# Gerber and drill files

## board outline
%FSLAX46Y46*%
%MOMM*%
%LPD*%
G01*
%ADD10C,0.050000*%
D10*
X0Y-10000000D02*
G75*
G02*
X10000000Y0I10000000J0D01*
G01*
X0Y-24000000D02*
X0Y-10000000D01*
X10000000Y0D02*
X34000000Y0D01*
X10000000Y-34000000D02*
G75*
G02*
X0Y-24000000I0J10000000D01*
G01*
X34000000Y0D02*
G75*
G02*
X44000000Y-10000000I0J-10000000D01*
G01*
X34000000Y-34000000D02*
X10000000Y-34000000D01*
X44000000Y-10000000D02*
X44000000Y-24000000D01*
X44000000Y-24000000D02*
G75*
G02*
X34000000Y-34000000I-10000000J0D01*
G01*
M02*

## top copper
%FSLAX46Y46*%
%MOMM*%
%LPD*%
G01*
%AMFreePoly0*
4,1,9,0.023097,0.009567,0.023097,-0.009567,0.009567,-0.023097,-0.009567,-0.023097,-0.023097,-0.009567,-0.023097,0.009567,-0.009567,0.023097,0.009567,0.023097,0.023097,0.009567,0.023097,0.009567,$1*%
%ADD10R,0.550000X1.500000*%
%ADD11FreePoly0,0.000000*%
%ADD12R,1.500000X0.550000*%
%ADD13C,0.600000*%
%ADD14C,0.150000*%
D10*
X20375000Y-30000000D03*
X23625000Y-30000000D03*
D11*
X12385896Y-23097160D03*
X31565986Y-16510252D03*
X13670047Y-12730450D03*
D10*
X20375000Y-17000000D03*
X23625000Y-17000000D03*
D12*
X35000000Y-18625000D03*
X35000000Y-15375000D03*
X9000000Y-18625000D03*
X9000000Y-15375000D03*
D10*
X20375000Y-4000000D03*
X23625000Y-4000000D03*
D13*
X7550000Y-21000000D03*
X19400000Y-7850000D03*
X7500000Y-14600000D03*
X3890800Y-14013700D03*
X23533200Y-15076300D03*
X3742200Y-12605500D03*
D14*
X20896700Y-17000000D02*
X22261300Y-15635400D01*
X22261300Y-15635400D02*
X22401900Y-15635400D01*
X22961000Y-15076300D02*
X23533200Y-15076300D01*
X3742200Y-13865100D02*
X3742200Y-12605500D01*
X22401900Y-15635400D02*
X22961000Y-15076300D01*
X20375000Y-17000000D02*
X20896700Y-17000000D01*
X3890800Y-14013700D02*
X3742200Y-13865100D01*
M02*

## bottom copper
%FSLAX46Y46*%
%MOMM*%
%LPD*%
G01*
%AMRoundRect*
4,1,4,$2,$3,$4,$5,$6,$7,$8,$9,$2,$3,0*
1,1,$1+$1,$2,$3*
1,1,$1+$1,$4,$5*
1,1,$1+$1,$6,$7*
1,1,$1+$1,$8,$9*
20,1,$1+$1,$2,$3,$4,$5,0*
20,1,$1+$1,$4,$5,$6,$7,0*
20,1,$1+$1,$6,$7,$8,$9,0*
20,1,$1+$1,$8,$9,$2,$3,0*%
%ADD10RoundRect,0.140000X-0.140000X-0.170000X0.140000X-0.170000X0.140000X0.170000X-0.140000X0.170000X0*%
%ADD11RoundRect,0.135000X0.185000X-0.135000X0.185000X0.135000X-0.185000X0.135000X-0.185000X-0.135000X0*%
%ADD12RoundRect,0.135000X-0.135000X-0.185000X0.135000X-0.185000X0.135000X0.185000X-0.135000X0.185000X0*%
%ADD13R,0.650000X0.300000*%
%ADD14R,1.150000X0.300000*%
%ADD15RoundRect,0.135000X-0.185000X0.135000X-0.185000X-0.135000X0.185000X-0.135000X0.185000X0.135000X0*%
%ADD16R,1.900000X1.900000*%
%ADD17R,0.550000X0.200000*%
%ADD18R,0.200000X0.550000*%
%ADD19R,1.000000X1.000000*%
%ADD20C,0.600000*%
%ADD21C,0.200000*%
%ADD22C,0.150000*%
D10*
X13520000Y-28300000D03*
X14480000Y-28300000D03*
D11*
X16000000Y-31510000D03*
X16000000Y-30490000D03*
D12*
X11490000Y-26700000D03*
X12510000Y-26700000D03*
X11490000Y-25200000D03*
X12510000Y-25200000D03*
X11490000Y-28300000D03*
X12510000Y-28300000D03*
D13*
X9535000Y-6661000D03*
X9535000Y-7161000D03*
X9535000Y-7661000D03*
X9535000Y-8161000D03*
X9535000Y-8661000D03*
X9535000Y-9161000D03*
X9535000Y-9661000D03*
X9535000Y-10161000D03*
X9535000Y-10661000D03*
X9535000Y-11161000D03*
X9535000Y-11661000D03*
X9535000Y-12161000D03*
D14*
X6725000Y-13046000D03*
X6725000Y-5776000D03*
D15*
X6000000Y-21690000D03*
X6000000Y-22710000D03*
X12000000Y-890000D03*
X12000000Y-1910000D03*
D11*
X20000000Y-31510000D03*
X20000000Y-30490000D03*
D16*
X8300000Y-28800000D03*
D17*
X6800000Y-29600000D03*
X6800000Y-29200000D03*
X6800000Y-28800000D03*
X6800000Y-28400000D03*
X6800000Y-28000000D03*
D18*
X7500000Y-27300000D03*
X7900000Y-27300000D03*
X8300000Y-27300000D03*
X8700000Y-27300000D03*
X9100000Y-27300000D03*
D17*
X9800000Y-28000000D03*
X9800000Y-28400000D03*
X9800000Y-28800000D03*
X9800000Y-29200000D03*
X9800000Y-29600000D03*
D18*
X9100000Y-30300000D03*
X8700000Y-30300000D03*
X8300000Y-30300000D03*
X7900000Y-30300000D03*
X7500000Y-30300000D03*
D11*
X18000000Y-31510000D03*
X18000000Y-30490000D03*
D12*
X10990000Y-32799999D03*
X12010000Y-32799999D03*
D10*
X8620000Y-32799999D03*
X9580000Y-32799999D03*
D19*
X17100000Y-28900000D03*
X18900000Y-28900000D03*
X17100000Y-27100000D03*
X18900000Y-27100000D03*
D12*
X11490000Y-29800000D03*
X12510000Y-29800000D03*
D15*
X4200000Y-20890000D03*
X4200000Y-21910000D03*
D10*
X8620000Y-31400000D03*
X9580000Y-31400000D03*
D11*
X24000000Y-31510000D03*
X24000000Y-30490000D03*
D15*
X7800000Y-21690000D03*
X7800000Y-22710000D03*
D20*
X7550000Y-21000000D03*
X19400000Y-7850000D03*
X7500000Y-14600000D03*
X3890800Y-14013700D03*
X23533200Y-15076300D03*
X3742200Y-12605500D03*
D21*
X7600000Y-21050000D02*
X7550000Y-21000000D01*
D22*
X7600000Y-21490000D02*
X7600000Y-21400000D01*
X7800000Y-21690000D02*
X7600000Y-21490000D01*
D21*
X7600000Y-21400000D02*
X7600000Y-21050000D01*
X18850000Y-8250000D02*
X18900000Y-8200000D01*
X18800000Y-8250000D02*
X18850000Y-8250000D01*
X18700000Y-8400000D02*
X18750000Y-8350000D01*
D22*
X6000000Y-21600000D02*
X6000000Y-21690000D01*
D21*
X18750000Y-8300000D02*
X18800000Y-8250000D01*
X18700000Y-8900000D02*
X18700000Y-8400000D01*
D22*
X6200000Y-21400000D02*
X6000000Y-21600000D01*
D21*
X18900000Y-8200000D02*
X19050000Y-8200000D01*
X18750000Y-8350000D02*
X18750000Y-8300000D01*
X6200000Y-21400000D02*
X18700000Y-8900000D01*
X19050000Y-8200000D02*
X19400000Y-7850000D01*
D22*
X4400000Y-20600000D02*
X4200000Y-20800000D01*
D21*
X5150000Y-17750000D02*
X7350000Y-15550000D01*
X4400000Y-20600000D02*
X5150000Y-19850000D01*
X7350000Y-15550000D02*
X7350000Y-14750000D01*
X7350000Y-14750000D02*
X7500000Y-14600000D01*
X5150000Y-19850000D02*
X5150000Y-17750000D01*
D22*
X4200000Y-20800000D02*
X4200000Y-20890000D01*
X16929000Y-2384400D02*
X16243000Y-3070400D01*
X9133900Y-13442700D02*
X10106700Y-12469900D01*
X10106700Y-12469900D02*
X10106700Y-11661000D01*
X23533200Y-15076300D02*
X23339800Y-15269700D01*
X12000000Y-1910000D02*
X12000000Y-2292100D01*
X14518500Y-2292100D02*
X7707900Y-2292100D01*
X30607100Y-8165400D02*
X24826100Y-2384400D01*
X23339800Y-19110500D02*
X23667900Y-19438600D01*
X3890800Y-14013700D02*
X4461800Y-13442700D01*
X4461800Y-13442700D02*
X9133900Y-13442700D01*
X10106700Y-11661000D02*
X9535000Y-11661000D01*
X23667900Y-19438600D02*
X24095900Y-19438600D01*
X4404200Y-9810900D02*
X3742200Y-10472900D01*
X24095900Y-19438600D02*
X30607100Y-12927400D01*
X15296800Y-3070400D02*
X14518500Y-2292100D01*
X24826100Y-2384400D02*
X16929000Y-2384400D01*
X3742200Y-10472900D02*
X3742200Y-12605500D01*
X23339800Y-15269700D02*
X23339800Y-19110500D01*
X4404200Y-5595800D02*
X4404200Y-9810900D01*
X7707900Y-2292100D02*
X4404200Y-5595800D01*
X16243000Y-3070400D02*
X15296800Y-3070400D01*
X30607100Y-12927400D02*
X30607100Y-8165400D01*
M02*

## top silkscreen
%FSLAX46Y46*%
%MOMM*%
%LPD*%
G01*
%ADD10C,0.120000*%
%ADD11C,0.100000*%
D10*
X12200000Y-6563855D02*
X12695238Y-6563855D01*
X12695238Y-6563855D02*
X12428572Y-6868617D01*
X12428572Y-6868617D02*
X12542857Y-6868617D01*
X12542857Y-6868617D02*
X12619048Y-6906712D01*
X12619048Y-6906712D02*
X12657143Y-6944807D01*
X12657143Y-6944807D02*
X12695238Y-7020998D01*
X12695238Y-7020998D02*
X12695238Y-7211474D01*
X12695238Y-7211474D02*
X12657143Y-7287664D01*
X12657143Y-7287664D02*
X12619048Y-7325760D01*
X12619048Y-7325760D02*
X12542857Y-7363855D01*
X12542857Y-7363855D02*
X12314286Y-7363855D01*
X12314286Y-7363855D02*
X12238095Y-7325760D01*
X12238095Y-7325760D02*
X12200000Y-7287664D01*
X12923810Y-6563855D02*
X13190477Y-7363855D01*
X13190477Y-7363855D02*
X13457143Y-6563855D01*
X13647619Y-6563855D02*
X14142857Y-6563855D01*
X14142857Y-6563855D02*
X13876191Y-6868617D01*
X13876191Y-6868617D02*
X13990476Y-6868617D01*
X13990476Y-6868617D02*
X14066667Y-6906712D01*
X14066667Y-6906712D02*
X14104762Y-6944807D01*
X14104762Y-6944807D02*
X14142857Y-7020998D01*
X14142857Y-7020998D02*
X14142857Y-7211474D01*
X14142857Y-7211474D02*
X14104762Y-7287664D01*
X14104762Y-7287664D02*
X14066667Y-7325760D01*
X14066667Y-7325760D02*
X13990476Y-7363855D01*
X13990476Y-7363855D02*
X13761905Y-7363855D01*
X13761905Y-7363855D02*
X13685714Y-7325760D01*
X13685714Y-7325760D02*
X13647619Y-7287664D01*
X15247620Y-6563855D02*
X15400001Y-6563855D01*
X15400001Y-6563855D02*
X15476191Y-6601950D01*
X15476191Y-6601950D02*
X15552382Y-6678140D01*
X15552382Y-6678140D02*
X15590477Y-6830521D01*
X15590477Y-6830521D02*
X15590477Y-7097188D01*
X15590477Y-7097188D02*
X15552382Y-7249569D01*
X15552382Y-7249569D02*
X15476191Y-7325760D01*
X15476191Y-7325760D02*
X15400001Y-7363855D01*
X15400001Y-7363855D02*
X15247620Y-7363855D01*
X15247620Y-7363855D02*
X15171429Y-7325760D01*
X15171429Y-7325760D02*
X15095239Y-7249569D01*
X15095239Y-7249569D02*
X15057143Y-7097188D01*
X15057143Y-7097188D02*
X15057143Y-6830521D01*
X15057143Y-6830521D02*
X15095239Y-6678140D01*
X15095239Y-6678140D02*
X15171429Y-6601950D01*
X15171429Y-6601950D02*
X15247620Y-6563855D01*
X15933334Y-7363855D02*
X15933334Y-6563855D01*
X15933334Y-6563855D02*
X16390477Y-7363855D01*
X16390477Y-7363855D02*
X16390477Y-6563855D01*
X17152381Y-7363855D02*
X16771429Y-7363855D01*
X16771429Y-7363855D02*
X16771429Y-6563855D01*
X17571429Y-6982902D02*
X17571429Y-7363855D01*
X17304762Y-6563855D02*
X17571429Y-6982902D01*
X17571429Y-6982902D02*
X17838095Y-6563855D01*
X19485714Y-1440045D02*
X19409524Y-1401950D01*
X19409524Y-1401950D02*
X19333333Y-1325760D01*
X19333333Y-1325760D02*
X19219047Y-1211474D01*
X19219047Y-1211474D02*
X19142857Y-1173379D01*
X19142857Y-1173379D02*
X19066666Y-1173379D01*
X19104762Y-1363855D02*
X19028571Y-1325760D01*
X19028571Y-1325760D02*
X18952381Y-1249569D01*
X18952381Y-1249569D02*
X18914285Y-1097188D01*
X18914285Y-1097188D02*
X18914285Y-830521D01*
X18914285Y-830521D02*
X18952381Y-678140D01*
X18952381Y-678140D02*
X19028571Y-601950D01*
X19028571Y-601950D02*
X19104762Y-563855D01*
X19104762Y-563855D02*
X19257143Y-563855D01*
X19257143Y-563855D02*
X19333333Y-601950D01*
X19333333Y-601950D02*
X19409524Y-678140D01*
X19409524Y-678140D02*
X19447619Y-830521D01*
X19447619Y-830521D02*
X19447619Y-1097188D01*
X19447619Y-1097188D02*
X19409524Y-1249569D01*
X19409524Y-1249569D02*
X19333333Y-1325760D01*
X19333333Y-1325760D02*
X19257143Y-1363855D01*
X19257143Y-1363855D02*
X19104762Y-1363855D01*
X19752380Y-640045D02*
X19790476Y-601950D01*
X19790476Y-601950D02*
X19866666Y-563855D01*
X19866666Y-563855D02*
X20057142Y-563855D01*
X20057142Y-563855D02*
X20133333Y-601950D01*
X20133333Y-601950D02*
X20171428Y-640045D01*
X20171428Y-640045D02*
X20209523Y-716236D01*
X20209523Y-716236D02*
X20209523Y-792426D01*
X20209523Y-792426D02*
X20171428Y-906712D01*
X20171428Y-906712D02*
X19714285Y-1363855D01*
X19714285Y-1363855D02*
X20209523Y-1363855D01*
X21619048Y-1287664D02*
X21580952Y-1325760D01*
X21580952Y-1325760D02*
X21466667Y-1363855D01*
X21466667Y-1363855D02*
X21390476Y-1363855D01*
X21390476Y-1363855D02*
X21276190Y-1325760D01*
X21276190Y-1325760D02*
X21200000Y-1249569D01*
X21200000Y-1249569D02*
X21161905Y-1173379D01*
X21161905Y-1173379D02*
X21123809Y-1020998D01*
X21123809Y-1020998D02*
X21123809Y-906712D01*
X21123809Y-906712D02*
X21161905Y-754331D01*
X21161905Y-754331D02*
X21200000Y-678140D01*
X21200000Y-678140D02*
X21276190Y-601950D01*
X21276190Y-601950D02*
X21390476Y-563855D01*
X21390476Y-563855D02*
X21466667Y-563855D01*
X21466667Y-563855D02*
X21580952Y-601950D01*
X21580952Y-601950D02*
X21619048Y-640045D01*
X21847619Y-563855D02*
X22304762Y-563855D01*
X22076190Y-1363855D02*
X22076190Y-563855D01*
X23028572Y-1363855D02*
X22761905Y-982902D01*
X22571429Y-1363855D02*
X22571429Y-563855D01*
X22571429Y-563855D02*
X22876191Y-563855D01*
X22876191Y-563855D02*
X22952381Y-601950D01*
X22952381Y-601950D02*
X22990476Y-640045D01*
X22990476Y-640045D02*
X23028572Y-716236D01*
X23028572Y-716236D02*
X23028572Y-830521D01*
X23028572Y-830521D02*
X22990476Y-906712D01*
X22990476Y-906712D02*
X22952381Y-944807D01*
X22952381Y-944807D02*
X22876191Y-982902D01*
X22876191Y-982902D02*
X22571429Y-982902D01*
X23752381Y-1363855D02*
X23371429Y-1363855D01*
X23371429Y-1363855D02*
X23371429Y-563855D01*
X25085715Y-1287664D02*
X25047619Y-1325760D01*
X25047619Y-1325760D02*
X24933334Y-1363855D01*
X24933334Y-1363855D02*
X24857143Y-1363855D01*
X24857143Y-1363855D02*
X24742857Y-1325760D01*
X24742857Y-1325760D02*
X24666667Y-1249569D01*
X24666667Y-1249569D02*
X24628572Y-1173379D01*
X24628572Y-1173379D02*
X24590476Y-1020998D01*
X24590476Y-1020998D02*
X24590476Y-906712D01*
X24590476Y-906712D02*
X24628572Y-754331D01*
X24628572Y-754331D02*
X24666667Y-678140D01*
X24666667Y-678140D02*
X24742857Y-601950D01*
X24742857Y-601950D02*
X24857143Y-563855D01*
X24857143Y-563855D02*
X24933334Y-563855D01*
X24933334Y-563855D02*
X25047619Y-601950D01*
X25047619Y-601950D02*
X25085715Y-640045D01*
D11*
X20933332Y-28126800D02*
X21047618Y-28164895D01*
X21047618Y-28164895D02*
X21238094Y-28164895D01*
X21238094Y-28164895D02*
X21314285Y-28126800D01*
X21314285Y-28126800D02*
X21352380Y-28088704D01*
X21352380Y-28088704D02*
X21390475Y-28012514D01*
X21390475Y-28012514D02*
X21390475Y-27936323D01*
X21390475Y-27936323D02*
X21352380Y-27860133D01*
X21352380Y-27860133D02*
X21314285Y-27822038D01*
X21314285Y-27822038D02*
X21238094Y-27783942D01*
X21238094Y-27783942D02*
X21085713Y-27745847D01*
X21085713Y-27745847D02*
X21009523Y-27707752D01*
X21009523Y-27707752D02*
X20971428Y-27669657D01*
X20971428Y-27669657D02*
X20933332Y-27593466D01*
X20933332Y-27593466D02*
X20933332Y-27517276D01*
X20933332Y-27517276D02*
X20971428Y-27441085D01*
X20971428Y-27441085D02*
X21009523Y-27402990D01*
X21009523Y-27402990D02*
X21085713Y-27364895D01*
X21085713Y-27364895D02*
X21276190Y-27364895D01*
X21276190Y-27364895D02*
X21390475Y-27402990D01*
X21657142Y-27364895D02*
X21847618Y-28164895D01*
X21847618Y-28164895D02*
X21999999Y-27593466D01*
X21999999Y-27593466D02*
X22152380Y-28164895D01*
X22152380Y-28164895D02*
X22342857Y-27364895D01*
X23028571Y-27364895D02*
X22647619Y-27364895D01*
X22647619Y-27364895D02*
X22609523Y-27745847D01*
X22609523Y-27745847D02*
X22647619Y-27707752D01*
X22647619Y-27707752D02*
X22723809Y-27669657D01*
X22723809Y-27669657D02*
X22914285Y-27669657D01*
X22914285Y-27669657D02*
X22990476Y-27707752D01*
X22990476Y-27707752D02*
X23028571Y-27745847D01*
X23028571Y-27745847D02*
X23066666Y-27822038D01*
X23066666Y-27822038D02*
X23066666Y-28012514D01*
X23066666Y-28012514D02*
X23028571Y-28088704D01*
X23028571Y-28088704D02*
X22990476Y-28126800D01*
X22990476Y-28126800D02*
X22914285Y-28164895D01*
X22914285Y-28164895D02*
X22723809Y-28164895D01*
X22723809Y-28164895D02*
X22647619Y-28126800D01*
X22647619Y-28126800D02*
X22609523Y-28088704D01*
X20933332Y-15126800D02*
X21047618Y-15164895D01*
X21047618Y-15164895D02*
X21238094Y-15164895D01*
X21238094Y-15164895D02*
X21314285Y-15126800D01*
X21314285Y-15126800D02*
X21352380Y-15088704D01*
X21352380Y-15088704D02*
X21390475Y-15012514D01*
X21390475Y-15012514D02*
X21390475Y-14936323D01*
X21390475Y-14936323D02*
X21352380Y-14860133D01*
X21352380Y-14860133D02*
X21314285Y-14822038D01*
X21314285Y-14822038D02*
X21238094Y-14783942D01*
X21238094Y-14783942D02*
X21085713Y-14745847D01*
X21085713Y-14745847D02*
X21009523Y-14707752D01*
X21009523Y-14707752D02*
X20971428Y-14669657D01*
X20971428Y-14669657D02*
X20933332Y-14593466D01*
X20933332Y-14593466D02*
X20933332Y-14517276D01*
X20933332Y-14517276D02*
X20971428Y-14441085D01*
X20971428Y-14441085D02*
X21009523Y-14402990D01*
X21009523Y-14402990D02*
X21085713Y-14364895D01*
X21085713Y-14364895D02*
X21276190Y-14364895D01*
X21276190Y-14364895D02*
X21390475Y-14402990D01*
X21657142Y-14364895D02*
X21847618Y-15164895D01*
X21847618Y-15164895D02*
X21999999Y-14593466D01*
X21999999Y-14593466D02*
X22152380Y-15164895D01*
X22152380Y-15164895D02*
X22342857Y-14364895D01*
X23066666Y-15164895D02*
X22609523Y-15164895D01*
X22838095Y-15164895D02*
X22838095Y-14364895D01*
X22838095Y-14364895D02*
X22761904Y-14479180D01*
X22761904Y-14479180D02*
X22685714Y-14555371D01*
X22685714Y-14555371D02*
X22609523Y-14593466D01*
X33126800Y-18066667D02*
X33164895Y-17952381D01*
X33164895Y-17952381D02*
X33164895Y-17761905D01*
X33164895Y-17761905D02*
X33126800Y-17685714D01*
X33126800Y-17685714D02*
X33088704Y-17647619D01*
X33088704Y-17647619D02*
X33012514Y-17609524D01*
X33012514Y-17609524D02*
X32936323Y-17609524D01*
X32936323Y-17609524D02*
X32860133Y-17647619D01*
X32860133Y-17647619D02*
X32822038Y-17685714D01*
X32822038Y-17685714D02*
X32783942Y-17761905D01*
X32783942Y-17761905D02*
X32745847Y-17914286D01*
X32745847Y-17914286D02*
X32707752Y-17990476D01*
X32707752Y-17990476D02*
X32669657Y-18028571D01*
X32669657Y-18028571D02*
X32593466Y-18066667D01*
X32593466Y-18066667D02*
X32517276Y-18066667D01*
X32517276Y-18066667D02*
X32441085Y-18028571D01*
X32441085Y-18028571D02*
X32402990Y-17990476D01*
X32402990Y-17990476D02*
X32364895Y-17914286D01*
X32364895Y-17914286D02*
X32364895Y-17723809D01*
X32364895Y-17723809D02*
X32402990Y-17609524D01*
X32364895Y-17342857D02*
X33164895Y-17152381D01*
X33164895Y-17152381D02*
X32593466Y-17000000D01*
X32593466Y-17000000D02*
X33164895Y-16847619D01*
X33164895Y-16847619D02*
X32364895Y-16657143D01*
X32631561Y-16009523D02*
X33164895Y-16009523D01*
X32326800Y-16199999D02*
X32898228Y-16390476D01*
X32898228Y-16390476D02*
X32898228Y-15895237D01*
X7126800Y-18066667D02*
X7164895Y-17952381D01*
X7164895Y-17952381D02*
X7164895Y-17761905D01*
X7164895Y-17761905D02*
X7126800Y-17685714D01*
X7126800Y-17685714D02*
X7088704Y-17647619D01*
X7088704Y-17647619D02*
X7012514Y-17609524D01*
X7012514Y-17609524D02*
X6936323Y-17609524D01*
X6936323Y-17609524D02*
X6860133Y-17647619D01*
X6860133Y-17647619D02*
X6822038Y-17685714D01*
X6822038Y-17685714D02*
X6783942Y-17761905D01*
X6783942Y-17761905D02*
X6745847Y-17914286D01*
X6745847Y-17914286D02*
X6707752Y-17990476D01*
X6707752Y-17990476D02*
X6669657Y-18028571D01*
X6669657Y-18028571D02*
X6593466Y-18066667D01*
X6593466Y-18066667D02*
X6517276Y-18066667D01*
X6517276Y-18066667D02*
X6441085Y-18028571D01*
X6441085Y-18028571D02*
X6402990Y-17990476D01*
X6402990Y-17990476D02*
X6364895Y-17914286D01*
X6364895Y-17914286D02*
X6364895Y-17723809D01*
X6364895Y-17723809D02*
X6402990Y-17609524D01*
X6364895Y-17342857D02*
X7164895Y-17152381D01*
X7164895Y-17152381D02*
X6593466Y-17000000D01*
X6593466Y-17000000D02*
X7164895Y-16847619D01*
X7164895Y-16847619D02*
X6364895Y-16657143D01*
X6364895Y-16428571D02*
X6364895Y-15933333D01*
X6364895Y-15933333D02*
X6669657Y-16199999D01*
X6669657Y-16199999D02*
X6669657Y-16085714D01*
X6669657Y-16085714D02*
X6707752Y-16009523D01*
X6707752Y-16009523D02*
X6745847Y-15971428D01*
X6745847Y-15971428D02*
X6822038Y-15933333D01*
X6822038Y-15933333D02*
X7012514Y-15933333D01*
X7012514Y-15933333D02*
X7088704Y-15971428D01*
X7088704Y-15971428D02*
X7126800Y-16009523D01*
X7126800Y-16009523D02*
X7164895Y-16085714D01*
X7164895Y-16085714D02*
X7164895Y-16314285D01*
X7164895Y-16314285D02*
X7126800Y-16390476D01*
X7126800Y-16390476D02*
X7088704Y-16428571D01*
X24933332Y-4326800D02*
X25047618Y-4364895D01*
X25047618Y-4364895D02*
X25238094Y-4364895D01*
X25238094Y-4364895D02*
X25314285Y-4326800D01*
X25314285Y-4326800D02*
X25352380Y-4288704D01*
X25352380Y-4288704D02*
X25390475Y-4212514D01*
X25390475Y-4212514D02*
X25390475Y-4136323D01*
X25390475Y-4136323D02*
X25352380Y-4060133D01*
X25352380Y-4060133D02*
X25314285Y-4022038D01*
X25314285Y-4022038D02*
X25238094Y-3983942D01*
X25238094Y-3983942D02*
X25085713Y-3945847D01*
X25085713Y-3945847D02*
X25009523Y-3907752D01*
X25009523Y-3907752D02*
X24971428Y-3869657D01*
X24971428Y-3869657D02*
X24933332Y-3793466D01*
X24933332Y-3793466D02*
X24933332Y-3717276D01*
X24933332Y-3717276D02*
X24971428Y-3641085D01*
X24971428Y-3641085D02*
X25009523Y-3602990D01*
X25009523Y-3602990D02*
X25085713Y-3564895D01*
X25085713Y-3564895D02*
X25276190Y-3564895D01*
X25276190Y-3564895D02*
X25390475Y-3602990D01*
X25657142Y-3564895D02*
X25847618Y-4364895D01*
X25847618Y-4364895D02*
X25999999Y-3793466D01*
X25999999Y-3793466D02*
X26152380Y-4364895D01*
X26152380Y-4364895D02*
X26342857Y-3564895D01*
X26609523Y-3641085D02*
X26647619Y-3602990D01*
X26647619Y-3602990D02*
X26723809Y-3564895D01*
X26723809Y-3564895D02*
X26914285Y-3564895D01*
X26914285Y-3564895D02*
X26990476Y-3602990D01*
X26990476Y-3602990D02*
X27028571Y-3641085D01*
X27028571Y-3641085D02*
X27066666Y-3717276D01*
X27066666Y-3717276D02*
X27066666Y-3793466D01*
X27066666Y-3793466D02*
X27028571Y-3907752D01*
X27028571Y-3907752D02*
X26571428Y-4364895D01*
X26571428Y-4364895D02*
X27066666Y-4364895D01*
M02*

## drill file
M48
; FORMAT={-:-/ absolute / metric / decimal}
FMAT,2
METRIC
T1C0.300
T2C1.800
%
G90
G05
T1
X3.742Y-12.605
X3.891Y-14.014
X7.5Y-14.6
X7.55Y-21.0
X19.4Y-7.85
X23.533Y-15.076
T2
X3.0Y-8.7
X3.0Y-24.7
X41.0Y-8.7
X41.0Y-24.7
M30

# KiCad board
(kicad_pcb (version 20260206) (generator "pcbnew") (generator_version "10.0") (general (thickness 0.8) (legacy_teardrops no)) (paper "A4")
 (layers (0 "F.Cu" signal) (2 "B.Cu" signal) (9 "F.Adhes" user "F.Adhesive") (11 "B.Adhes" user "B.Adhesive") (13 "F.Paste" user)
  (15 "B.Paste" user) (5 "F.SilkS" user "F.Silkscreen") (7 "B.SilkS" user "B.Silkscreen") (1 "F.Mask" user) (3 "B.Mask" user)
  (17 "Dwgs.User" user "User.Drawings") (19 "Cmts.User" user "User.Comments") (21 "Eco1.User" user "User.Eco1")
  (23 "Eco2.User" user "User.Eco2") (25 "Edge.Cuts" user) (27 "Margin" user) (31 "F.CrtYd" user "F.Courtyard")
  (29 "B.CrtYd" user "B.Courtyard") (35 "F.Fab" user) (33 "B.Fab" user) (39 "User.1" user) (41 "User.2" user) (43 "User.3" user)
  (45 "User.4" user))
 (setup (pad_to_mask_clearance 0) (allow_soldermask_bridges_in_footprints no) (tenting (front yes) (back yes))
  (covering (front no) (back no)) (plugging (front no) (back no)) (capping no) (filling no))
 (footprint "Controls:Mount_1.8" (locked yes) (layer "F.Cu") (at 41 24.7)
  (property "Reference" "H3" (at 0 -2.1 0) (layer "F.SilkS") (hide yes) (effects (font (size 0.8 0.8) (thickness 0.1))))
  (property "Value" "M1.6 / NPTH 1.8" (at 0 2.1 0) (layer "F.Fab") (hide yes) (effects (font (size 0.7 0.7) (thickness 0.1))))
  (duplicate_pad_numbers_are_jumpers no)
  (pad "" np_thru_hole circle (at 0 0) (size 1.8 1.8) (drill 1.8) (layers "*.Cu" "*.Mask")))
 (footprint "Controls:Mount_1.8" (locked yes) (layer "F.Cu") (at 3 8.7)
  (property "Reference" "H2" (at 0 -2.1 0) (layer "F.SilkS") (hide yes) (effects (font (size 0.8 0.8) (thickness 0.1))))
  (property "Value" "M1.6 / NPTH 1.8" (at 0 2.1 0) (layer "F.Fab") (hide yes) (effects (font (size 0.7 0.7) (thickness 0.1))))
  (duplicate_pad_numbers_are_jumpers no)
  (pad "" np_thru_hole circle (at 0 0) (size 1.8 1.8) (drill 1.8) (layers "*.Cu" "*.Mask")))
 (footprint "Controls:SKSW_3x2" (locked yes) (layer "F.Cu") (at 22 30)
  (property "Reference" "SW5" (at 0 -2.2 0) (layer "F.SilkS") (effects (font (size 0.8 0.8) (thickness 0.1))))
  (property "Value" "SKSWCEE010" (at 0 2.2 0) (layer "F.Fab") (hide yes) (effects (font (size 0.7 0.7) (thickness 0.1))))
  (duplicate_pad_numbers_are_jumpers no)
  (pad "1" smd rect (at -1.625 0) (size 0.55 1.5) (layers "F.Cu" "F.Mask" "F.Paste") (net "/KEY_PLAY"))
  (pad "2" smd rect (at 1.625 0) (size 0.55 1.5) (layers "F.Cu" "F.Mask" "F.Paste") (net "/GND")))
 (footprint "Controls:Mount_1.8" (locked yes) (layer "F.Cu") (at 41 8.7)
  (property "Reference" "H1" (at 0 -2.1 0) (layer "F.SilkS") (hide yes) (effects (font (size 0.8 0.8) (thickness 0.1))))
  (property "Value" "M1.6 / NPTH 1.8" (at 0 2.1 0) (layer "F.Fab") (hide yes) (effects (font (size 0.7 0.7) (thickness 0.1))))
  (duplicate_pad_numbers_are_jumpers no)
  (pad "" np_thru_hole circle (at 0 0) (size 1.8 1.8) (drill 1.8) (layers "*.Cu" "*.Mask")))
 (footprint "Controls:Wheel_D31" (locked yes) (layer "F.Cu") (at 22 17)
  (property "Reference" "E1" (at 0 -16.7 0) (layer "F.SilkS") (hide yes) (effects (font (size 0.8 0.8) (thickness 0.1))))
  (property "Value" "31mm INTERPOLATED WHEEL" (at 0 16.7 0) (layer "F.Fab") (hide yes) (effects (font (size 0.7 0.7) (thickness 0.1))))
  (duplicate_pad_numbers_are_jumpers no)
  (pad "1" smd custom (at -9.614104 6.09716) (size 0.05 0.05) (layers "F.Cu") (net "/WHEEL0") (options (clearance outline) (anchor circle))
   (primitives))
  (pad "2" smd custom (at 9.565986 -0.489748) (size 0.05 0.05) (layers "F.Cu") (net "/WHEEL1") (options (clearance outline) (anchor circle))
   (primitives))
  (pad "3" smd custom (at -8.329953 -4.26955) (size 0.05 0.05) (layers "F.Cu") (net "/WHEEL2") (options (clearance outline) (anchor circle))
   (primitives)))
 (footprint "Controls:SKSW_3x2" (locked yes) (layer "F.Cu") (at 22 17)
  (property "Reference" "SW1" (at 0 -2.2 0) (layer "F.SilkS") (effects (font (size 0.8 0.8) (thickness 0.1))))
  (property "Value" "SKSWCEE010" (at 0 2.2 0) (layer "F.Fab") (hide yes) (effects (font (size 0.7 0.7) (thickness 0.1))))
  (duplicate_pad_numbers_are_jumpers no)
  (pad "1" smd rect (at -1.625 0) (size 0.55 1.5) (layers "F.Cu" "F.Mask" "F.Paste") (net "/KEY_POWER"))
  (pad "2" smd rect (at 1.625 0) (size 0.55 1.5) (layers "F.Cu" "F.Mask" "F.Paste") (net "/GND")))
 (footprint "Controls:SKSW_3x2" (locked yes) (layer "F.Cu") (at 35 17 90)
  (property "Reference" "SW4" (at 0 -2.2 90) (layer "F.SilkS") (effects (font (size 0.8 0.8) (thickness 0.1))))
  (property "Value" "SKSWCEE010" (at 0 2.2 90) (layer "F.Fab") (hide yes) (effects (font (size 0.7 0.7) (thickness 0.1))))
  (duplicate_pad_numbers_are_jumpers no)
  (pad "1" smd rect (at -1.625 0 90) (size 0.55 1.5) (layers "F.Cu" "F.Mask" "F.Paste") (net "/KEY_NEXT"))
  (pad "2" smd rect (at 1.625 0 90) (size 0.55 1.5) (layers "F.Cu" "F.Mask" "F.Paste") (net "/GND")))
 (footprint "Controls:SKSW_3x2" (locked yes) (layer "F.Cu") (at 9 17 90)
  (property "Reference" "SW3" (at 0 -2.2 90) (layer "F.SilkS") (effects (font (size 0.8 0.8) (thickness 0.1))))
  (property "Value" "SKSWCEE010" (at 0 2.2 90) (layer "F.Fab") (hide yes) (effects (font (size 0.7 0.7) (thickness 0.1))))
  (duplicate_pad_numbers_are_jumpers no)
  (pad "1" smd rect (at -1.625 0 90) (size 0.55 1.5) (layers "F.Cu" "F.Mask" "F.Paste") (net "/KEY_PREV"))
  (pad "2" smd rect (at 1.625 0 90) (size 0.55 1.5) (layers "F.Cu" "F.Mask" "F.Paste") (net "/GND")))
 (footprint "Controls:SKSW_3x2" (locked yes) (layer "F.Cu") (at 22 4)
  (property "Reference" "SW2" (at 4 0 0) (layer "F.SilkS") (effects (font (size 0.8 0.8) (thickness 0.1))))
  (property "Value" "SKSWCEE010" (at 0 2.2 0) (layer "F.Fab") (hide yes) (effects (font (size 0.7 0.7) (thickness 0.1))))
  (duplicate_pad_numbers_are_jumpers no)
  (pad "1" smd rect (at -1.625 0) (size 0.55 1.5) (layers "F.Cu" "F.Mask" "F.Paste") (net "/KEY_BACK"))
  (pad "2" smd rect (at 1.625 0) (size 0.55 1.5) (layers "F.Cu" "F.Mask" "F.Paste") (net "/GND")))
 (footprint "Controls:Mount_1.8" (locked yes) (layer "F.Cu") (at 3 24.7)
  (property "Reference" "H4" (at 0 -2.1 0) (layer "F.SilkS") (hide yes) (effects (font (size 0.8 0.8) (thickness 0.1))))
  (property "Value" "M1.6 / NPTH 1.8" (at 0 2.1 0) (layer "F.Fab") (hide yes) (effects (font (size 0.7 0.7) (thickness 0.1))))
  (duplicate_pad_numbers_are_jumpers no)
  (pad "" np_thru_hole circle (at 0 0) (size 1.8 1.8) (drill 1.8) (layers "*.Cu" "*.Mask")))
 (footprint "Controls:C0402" (layer "B.Cu") (at 14 28.3)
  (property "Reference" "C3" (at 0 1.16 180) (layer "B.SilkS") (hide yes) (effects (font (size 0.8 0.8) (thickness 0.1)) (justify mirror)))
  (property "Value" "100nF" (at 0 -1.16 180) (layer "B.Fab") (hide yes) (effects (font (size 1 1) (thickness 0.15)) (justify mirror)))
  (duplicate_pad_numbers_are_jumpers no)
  (pad "1" smd roundrect (at -0.48 0) (size 0.56 0.62) (layers "B.Cu" "B.Mask" "B.Paste") (roundrect_rratio 0.25) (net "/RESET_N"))
  (pad "2" smd roundrect (at 0.48 0) (size 0.56 0.62) (layers "B.Cu" "B.Mask" "B.Paste") (roundrect_rratio 0.25) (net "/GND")))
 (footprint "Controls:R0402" (layer "B.Cu") (at 16 31 90)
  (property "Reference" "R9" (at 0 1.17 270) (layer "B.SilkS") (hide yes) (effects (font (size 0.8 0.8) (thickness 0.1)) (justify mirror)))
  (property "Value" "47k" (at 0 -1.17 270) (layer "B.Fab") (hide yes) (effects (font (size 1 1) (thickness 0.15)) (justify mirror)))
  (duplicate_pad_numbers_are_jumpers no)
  (pad "1" smd roundrect (at -0.51 0 90) (size 0.54 0.64) (layers "B.Cu" "B.Mask" "B.Paste") (roundrect_rratio 0.25) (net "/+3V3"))
  (pad "2" smd roundrect (at 0.51 0 90) (size 0.54 0.64) (layers "B.Cu" "B.Mask" "B.Paste") (roundrect_rratio 0.25) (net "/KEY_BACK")))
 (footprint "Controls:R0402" (layer "B.Cu") (at 12 26.7)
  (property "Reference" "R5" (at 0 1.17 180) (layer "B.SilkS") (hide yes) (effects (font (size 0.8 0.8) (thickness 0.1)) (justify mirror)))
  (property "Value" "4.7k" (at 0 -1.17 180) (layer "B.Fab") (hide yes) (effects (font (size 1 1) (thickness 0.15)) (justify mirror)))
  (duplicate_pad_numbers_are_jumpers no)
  (pad "1" smd roundrect (at -0.51 0) (size 0.54 0.64) (layers "B.Cu" "B.Mask" "B.Paste") (roundrect_rratio 0.25) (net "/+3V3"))
  (pad "2" smd roundrect (at 0.51 0) (size 0.54 0.64) (layers "B.Cu" "B.Mask" "B.Paste") (roundrect_rratio 0.25) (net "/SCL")))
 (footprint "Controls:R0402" (layer "B.Cu") (at 12 25.2)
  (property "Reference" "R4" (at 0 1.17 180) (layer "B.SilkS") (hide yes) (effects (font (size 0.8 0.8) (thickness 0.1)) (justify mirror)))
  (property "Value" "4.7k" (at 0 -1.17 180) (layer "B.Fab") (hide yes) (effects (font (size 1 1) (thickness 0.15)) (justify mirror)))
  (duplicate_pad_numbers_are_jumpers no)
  (pad "1" smd roundrect (at -0.51 0) (size 0.54 0.64) (layers "B.Cu" "B.Mask" "B.Paste") (roundrect_rratio 0.25) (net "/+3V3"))
  (pad "2" smd roundrect (at 0.51 0) (size 0.54 0.64) (layers "B.Cu" "B.Mask" "B.Paste") (roundrect_rratio 0.25) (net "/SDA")))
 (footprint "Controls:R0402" (layer "B.Cu") (at 12 28.3)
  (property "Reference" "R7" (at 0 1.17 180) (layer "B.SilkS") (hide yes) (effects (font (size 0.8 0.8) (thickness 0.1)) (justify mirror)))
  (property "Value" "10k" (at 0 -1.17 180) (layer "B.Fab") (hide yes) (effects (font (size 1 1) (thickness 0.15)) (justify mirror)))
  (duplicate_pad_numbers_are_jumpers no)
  (pad "1" smd roundrect (at -0.51 0) (size 0.54 0.64) (layers "B.Cu" "B.Mask" "B.Paste") (roundrect_rratio 0.25) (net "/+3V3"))
  (pad "2" smd roundrect (at 0.51 0) (size 0.54 0.64) (layers "B.Cu" "B.Mask" "B.Paste") (roundrect_rratio 0.25) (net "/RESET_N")))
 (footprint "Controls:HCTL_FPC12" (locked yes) (layer "B.Cu") (at 8.13 9.411 -90)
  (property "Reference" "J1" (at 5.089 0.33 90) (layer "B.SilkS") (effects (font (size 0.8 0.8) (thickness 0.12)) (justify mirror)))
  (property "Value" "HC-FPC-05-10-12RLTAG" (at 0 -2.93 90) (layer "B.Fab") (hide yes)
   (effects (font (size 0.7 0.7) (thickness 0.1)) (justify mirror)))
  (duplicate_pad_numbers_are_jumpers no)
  (pad "1" smd rect (at -2.75 -1.405 270) (size 0.3 0.65) (layers "B.Cu" "B.Mask" "B.Paste") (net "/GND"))
  (pad "2" smd rect (at -2.25 -1.405 270) (size 0.3 0.65) (layers "B.Cu" "B.Mask" "B.Paste") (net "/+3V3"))
  (pad "3" smd rect (at -1.75 -1.405 270) (size 0.3 0.65) (layers "B.Cu" "B.Mask" "B.Paste") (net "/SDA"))
  (pad "4" smd rect (at -1.25 -1.405 270) (size 0.3 0.65) (layers "B.Cu" "B.Mask" "B.Paste") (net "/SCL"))
  (pad "5" smd rect (at -0.75 -1.405 270) (size 0.3 0.65) (layers "B.Cu" "B.Mask" "B.Paste") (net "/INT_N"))
  (pad "6" smd rect (at -0.25 -1.405 270) (size 0.3 0.65) (layers "B.Cu" "B.Mask" "B.Paste") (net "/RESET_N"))
  (pad "7" smd rect (at 0.25 -1.405 270) (size 0.3 0.65) (layers "B.Cu" "B.Mask" "B.Paste") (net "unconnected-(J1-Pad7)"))
  (pad "8" smd rect (at 0.75 -1.405 270) (size 0.3 0.65) (layers "B.Cu" "B.Mask" "B.Paste") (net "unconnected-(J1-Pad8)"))
  (pad "9" smd rect (at 1.25 -1.405 270) (size 0.3 0.65) (layers "B.Cu" "B.Mask" "B.Paste") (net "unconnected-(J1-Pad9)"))
  (pad "10" smd rect (at 1.75 -1.405 270) (size 0.3 0.65) (layers "B.Cu" "B.Mask" "B.Paste") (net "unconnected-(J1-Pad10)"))
  (pad "11" smd rect (at 2.25 -1.405 270) (size 0.3 0.65) (layers "B.Cu" "B.Mask" "B.Paste") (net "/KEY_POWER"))
  (pad "12" smd rect (at 2.75 -1.405 270) (size 0.3 0.65) (layers "B.Cu" "B.Mask" "B.Paste") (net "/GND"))
  (pad "13" smd rect (at 3.635 1.405 270) (size 0.3 1.15) (layers "B.Cu" "B.Mask" "B.Paste") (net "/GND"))
  (pad "14" smd rect (at -3.635 1.405 270) (size 0.3 1.15) (layers "B.Cu" "B.Mask" "B.Paste") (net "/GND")))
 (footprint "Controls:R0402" (layer "B.Cu") (at 6 22.2 -90)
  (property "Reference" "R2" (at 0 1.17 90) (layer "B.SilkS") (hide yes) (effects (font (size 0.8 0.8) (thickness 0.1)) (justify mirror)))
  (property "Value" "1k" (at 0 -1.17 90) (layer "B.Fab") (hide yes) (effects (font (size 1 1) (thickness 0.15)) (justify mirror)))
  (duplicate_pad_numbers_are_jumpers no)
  (pad "1" smd roundrect (at -0.51 0 270) (size 0.54 0.64) (layers "B.Cu" "B.Mask" "B.Paste") (roundrect_rratio 0.25) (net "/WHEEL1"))
  (pad "2" smd roundrect (at 0.51 0 270) (size 0.54 0.64) (layers "B.Cu" "B.Mask" "B.Paste") (roundrect_rratio 0.25) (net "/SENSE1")))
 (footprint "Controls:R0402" (layer "B.Cu") (at 12 1.4 -90)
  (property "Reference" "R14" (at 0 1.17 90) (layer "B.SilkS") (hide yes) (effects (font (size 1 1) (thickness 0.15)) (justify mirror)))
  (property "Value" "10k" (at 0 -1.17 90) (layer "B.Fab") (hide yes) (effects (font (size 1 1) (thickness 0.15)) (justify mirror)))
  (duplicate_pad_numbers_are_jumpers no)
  (pad "1" smd roundrect (at -0.51 0 270) (size 0.54 0.64) (layers "B.Cu" "B.Mask" "B.Paste") (roundrect_rratio 0.25) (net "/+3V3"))
  (pad "2" smd roundrect (at 0.51 0 270) (size 0.54 0.64) (layers "B.Cu" "B.Mask" "B.Paste") (roundrect_rratio 0.25) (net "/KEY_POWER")))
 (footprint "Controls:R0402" (layer "B.Cu") (at 20 31 90)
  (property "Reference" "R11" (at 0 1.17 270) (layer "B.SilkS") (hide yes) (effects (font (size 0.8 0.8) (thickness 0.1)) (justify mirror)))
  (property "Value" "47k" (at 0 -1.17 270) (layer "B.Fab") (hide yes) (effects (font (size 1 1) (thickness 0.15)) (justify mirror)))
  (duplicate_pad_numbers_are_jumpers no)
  (pad "1" smd roundrect (at -0.51 0 90) (size 0.54 0.64) (layers "B.Cu" "B.Mask" "B.Paste") (roundrect_rratio 0.25) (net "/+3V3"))
  (pad "2" smd roundrect (at 0.51 0 90) (size 0.54 0.64) (layers "B.Cu" "B.Mask" "B.Paste") (roundrect_rratio 0.25) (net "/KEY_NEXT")))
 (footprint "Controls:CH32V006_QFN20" (layer "B.Cu") (at 8.3 28.8)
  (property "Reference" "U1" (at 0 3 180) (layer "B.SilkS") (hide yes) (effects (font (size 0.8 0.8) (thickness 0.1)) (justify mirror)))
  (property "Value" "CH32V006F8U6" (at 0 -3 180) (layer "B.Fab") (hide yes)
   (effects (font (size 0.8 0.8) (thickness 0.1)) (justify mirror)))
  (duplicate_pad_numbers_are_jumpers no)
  (pad "" smd rect (at -0.45 -0.45) (size 0.7 0.7) (layers "B.Paste"))
  (pad "" smd rect (at -0.45 0.45) (size 0.7 0.7) (layers "B.Paste"))
  (pad "" smd rect (at 0.45 -0.45) (size 0.7 0.7) (layers "B.Paste"))
  (pad "" smd rect (at 0.45 0.45) (size 0.7 0.7) (layers "B.Paste"))
  (pad "0" smd rect (at 0 0) (size 1.9 1.9) (layers "B.Cu" "B.Mask") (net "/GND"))
  (pad "1" smd rect (at -1.5 0.8) (size 0.55 0.2) (layers "B.Cu" "B.Mask" "B.Paste") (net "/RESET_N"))
  (pad "2" smd rect (at -1.5 0.4) (size 0.55 0.2) (layers "B.Cu" "B.Mask" "B.Paste") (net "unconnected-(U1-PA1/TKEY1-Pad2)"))
  (pad "3" smd rect (at -1.5 0) (size 0.55 0.2) (layers "B.Cu" "B.Mask" "B.Paste") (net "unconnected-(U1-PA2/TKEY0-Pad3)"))
  (pad "4" smd rect (at -1.5 -0.4) (size 0.55 0.2) (layers "B.Cu" "B.Mask" "B.Paste") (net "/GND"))
  (pad "5" smd rect (at -1.5 -0.8) (size 0.55 0.2) (layers "B.Cu" "B.Mask" "B.Paste") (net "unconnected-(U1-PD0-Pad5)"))
  (pad "6" smd rect (at -0.8 -1.5) (size 0.2 0.55) (layers "B.Cu" "B.Mask" "B.Paste") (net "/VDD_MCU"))
  (pad "7" smd rect (at -0.4 -1.5) (size 0.2 0.55) (layers "B.Cu" "B.Mask" "B.Paste") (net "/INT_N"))
  (pad "8" smd rect (at 0 -1.5) (size 0.2 0.55) (layers "B.Cu" "B.Mask" "B.Paste") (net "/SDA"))
  (pad "9" smd rect (at 0.4 -1.5) (size 0.2 0.55) (layers "B.Cu" "B.Mask" "B.Paste") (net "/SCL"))
  (pad "10" smd rect (at 0.8 -1.5) (size 0.2 0.55) (layers "B.Cu" "B.Mask" "B.Paste") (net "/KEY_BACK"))
  (pad "11" smd rect (at 1.5 -0.8) (size 0.55 0.2) (layers "B.Cu" "B.Mask" "B.Paste") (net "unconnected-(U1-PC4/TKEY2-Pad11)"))
  (pad "12" smd rect (at 1.5 -0.4) (size 0.55 0.2) (layers "B.Cu" "B.Mask" "B.Paste") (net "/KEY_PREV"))
  (pad "13" smd rect (at 1.5 0) (size 0.55 0.2) (layers "B.Cu" "B.Mask" "B.Paste") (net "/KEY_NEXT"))
  (pad "14" smd rect (at 1.5 0.4) (size 0.55 0.2) (layers "B.Cu" "B.Mask" "B.Paste") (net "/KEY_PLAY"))
  (pad "15" smd rect (at 1.5 0.8) (size 0.55 0.2) (layers "B.Cu" "B.Mask" "B.Paste") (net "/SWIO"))
  (pad "16" smd rect (at 0.8 1.5) (size 0.2 0.55) (layers "B.Cu" "B.Mask" "B.Paste") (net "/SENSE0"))
  (pad "17" smd rect (at 0.4 1.5) (size 0.2 0.55) (layers "B.Cu" "B.Mask" "B.Paste") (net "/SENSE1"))
  (pad "18" smd rect (at 0 1.5) (size 0.2 0.55) (layers "B.Cu" "B.Mask" "B.Paste") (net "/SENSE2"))
  (pad "19" smd rect (at -0.4 1.5) (size 0.2 0.55) (layers "B.Cu" "B.Mask" "B.Paste") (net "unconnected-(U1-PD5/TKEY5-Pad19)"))
  (pad "20" smd rect (at -0.8 1.5) (size 0.2 0.55) (layers "B.Cu" "B.Mask" "B.Paste") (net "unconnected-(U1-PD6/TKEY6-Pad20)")))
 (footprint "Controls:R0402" (layer "B.Cu") (at 18 31 90)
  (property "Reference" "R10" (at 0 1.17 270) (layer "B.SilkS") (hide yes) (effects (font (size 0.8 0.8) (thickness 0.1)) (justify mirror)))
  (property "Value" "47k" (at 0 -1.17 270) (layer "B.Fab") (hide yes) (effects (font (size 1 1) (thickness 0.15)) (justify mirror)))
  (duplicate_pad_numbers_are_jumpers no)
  (pad "1" smd roundrect (at -0.51 0 90) (size 0.54 0.64) (layers "B.Cu" "B.Mask" "B.Paste") (roundrect_rratio 0.25) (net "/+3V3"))
  (pad "2" smd roundrect (at 0.51 0 90) (size 0.54 0.64) (layers "B.Cu" "B.Mask" "B.Paste") (roundrect_rratio 0.25) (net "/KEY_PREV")))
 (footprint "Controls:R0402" (layer "B.Cu") (at 11.5 32.799999)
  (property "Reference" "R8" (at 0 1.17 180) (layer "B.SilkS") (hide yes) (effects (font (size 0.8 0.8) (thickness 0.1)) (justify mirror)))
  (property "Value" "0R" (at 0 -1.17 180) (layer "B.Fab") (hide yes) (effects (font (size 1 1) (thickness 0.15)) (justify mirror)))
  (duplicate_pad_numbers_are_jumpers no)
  (pad "1" smd roundrect (at -0.51 0) (size 0.54 0.64) (layers "B.Cu" "B.Mask" "B.Paste") (roundrect_rratio 0.25) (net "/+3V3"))
  (pad "2" smd roundrect (at 0.51 0) (size 0.54 0.64) (layers "B.Cu" "B.Mask" "B.Paste") (roundrect_rratio 0.25) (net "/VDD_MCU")))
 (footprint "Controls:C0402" (layer "B.Cu") (at 9.1 32.799999)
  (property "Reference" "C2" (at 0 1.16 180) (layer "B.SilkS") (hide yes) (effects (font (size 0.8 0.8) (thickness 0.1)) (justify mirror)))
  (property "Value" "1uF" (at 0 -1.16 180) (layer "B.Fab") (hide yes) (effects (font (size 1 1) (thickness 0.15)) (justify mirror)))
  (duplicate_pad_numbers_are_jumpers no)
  (pad "1" smd roundrect (at -0.48 0) (size 0.56 0.62) (layers "B.Cu" "B.Mask" "B.Paste") (roundrect_rratio 0.25) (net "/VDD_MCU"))
  (pad "2" smd roundrect (at 0.48 0) (size 0.56 0.62) (layers "B.Cu" "B.Mask" "B.Paste") (roundrect_rratio 0.25) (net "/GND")))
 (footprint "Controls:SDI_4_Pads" (layer "B.Cu") (at 18 28)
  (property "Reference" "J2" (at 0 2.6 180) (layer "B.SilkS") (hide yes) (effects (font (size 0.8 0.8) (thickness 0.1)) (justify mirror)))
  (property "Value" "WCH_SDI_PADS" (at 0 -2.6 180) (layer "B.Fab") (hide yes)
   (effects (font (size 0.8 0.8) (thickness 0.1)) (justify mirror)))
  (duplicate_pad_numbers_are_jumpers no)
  (pad "1" smd rect (at -0.9 0.9) (size 1 1) (layers "B.Cu" "B.Mask") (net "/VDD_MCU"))
  (pad "2" smd rect (at 0.9 0.9) (size 1 1) (layers "B.Cu" "B.Mask") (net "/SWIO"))
  (pad "3" smd rect (at -0.9 -0.9) (size 1 1) (layers "B.Cu" "B.Mask") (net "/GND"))
  (pad "4" smd rect (at 0.9 -0.9) (size 1 1) (layers "B.Cu" "B.Mask") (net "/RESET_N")))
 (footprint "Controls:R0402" (layer "B.Cu") (at 12 29.8)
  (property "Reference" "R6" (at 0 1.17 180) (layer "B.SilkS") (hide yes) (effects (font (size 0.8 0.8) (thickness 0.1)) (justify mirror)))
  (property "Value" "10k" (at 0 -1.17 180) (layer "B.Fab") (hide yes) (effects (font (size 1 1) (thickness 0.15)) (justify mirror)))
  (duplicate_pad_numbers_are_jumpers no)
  (pad "1" smd roundrect (at -0.51 0) (size 0.54 0.64) (layers "B.Cu" "B.Mask" "B.Paste") (roundrect_rratio 0.25) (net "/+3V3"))
  (pad "2" smd roundrect (at 0.51 0) (size 0.54 0.64) (layers "B.Cu" "B.Mask" "B.Paste") (roundrect_rratio 0.25) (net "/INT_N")))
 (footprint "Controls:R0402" (layer "B.Cu") (at 4.2 21.4 -90)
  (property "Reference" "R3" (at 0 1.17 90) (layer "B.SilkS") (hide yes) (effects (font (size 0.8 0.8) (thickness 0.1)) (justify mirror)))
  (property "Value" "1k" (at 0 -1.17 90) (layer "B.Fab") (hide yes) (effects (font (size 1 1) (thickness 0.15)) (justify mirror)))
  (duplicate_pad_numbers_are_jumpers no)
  (pad "1" smd roundrect (at -0.51 0 270) (size 0.54 0.64) (layers "B.Cu" "B.Mask" "B.Paste") (roundrect_rratio 0.25) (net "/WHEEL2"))
  (pad "2" smd roundrect (at 0.51 0 270) (size 0.54 0.64) (layers "B.Cu" "B.Mask" "B.Paste") (roundrect_rratio 0.25) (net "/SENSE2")))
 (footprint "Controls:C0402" (layer "B.Cu") (at 9.1 31.4)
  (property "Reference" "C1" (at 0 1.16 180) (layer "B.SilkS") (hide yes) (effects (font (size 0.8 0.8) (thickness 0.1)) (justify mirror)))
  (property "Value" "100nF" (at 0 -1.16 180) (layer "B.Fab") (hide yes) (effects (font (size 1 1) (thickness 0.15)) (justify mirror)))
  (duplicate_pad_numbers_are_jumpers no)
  (pad "1" smd roundrect (at -0.48 0) (size 0.56 0.62) (layers "B.Cu" "B.Mask" "B.Paste") (roundrect_rratio 0.25) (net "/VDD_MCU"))
  (pad "2" smd roundrect (at 0.48 0) (size 0.56 0.62) (layers "B.Cu" "B.Mask" "B.Paste") (roundrect_rratio 0.25) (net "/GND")))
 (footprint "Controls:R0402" (layer "B.Cu") (at 24 31 90)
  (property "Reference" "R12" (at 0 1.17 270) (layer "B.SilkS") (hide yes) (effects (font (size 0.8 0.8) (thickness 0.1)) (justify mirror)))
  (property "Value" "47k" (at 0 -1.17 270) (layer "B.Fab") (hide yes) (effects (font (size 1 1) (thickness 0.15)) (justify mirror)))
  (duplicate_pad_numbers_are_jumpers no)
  (pad "1" smd roundrect (at -0.51 0 90) (size 0.54 0.64) (layers "B.Cu" "B.Mask" "B.Paste") (roundrect_rratio 0.25) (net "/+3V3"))
  (pad "2" smd roundrect (at 0.51 0 90) (size 0.54 0.64) (layers "B.Cu" "B.Mask" "B.Paste") (roundrect_rratio 0.25) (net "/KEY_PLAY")))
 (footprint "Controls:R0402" (layer "B.Cu") (at 7.8 22.2 -90)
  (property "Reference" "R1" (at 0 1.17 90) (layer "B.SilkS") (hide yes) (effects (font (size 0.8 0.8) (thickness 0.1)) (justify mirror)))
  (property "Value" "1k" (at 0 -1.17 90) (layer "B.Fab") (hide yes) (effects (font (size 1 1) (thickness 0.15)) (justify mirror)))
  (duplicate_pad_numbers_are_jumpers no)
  (pad "1" smd roundrect (at -0.51 0 270) (size 0.54 0.64) (layers "B.Cu" "B.Mask" "B.Paste") (roundrect_rratio 0.25) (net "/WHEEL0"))
  (pad "2" smd roundrect (at 0.51 0 270) (size 0.54 0.64) (layers "B.Cu" "B.Mask" "B.Paste") (roundrect_rratio 0.25) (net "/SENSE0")))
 (gr_arc (start 0 10) (mid 2.928932 2.928932) (end 10 0) (stroke (width 0.05) (type default)) (layer "Edge.Cuts"))
 (gr_line (start 0 24) (end 0 10) (stroke (width 0.05) (type default)) (layer "Edge.Cuts"))
 (gr_line (start 10 0) (end 34 0) (stroke (width 0.05) (type default)) (layer "Edge.Cuts"))
 (gr_arc (start 10 34) (mid 2.928932 31.071068) (end 0 24) (stroke (width 0.05) (type default)) (layer "Edge.Cuts"))
 (gr_arc (start 34 0) (mid 41.071068 2.928932) (end 44 10) (stroke (width 0.05) (type default)) (layer "Edge.Cuts"))
 (gr_line (start 34 34) (end 10 34) (stroke (width 0.05) (type default)) (layer "Edge.Cuts"))
 (gr_line (start 44 10) (end 44 24) (stroke (width 0.05) (type default)) (layer "Edge.Cuts"))
 (gr_arc (start 44 24) (mid 41.071068 31.071068) (end 34 34) (stroke (width 0.05) (type default)) (layer "Edge.Cuts"))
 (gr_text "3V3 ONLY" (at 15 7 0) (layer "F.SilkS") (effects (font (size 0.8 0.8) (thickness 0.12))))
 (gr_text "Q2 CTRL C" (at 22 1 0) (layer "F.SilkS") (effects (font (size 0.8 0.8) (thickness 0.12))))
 (via (at 7.55 21) (size 0.6) (drill 0.3) (layers "F.Cu" "B.Cu") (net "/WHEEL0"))
 (segment (start 7.6 21.05) (end 7.55 21) (width 0.2) (layer "B.Cu") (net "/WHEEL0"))
 (segment (start 7.6 21.49) (end 7.6 21.4) (width 0.15) (layer "B.Cu") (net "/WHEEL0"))
 (segment (start 7.8 21.69) (end 7.6 21.49) (width 0.15) (layer "B.Cu") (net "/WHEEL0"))
 (segment (start 7.6 21.4) (end 7.6 21.05) (width 0.2) (layer "B.Cu") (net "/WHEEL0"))
 (via (at 19.4 7.85) (size 0.6) (drill 0.3) (layers "F.Cu" "B.Cu") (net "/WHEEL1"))
 (segment (start 18.85 8.25) (end 18.9 8.2) (width 0.2) (layer "B.Cu") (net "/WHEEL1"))
 (segment (start 18.8 8.25) (end 18.85 8.25) (width 0.2) (layer "B.Cu") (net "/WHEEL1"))
 (segment (start 18.7 8.4) (end 18.75 8.35) (width 0.2) (layer "B.Cu") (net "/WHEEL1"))
 (segment (start 6 21.6) (end 6 21.69) (width 0.15) (layer "B.Cu") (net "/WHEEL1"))
 (segment (start 18.75 8.3) (end 18.8 8.25) (width 0.2) (layer "B.Cu") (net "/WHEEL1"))
 (segment (start 18.7 8.9) (end 18.7 8.4) (width 0.2) (layer "B.Cu") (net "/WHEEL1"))
 (segment (start 6.2 21.4) (end 6 21.6) (width 0.15) (layer "B.Cu") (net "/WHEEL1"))
 (segment (start 18.9 8.2) (end 19.05 8.2) (width 0.2) (layer "B.Cu") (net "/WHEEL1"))
 (segment (start 18.75 8.35) (end 18.75 8.3) (width 0.2) (layer "B.Cu") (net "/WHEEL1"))
 (segment (start 6.2 21.4) (end 18.7 8.9) (width 0.2) (layer "B.Cu") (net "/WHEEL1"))
 (segment (start 19.05 8.2) (end 19.4 7.85) (width 0.2) (layer "B.Cu") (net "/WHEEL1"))
 (via (at 7.5 14.6) (size 0.6) (drill 0.3) (layers "F.Cu" "B.Cu") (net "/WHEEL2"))
 (segment (start 4.4 20.6) (end 4.2 20.8) (width 0.15) (layer "B.Cu") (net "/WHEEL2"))
 (segment (start 5.15 17.75) (end 7.35 15.55) (width 0.2) (layer "B.Cu") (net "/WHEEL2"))
 (segment (start 4.4 20.6) (end 5.15 19.85) (width 0.2) (layer "B.Cu") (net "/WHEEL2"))
 (segment (start 7.35 15.55) (end 7.35 14.75) (width 0.2) (layer "B.Cu") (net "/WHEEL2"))
 (segment (start 7.35 14.75) (end 7.5 14.6) (width 0.2) (layer "B.Cu") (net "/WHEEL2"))
 (segment (start 5.15 19.85) (end 5.15 17.75) (width 0.2) (layer "B.Cu") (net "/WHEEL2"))
 (segment (start 4.2 20.8) (end 4.2 20.89) (width 0.15) (layer "B.Cu") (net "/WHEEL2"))
 (segment (start 20.8967 17) (end 22.2613 15.6354) (width 0.15) (layer "F.Cu") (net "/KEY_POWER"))
 (segment (start 22.2613 15.6354) (end 22.4019 15.6354) (width 0.15) (layer "F.Cu") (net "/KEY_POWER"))
 (segment (start 22.961 15.0763) (end 23.5332 15.0763) (width 0.15) (layer "F.Cu") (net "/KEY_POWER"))
 (segment (start 3.7422 13.8651) (end 3.7422 12.6055) (width 0.15) (layer "F.Cu") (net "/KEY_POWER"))
 (segment (start 22.4019 15.6354) (end 22.961 15.0763) (width 0.15) (layer "F.Cu") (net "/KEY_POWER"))
 (segment (start 20.375 17) (end 20.8967 17) (width 0.15) (layer "F.Cu") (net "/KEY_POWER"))
 (segment (start 3.8908 14.0137) (end 3.7422 13.8651) (width 0.15) (layer "F.Cu") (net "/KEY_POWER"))
 (via (at 3.8908 14.0137) (size 0.6) (drill 0.3) (layers "F.Cu" "B.Cu") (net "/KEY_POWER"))
 (via (at 23.5332 15.0763) (size 0.6) (drill 0.3) (layers "F.Cu" "B.Cu") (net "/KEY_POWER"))
 (via (at 3.7422 12.6055) (size 0.6) (drill 0.3) (layers "F.Cu" "B.Cu") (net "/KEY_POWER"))
 (segment (start 16.929 2.3844) (end 16.243 3.0704) (width 0.15) (layer "B.Cu") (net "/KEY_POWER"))
 (segment (start 9.1339 13.4427) (end 10.1067 12.4699) (width 0.15) (layer "B.Cu") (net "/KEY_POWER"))
 (segment (start 10.1067 12.4699) (end 10.1067 11.661) (width 0.15) (layer "B.Cu") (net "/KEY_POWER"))
 (segment (start 23.5332 15.0763) (end 23.3398 15.2697) (width 0.15) (layer "B.Cu") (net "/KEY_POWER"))
 (segment (start 12 1.91) (end 12 2.2921) (width 0.15) (layer "B.Cu") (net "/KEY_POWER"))
 (segment (start 14.5185 2.2921) (end 7.7079 2.2921) (width 0.15) (layer "B.Cu") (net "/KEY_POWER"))
 (segment (start 30.6071 8.1654) (end 24.8261 2.3844) (width 0.15) (layer "B.Cu") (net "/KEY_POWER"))
 (segment (start 23.3398 19.1105) (end 23.6679 19.4386) (width 0.15) (layer "B.Cu") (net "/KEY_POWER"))
 (segment (start 3.8908 14.0137) (end 4.4618 13.4427) (width 0.15) (layer "B.Cu") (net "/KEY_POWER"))
 (segment (start 4.4618 13.4427) (end 9.1339 13.4427) (width 0.15) (layer "B.Cu") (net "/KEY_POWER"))
 (segment (start 10.1067 11.661) (end 9.535 11.661) (width 0.15) (layer "B.Cu") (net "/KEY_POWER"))
 (segment (start 23.6679 19.4386) (end 24.0959 19.4386) (width 0.15) (layer "B.Cu") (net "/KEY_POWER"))
 (segment (start 4.4042 9.8109) (end 3.7422 10.4729) (width 0.15) (layer "B.Cu") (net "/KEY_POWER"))
 (segment (start 24.0959 19.4386) (end 30.6071 12.9274) (width 0.15) (layer "B.Cu") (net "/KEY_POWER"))
 (segment (start 15.2968 3.0704) (end 14.5185 2.2921) (width 0.15) (layer "B.Cu") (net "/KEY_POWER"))
 (segment (start 24.8261 2.3844) (end 16.929 2.3844) (width 0.15) (layer "B.Cu") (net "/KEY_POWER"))
 (segment (start 3.7422 10.4729) (end 3.7422 12.6055) (width 0.15) (layer "B.Cu") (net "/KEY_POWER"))
 (segment (start 23.3398 15.2697) (end 23.3398 19.1105) (width 0.15) (layer "B.Cu") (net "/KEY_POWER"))
 (segment (start 4.4042 5.5958) (end 4.4042 9.8109) (width 0.15) (layer "B.Cu") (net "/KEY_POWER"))
 (segment (start 7.7079 2.2921) (end 4.4042 5.5958) (width 0.15) (layer "B.Cu") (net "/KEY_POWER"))
 (segment (start 16.243 3.0704) (end 15.2968 3.0704) (width 0.15) (layer "B.Cu") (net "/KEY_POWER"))
 (segment (start 30.6071 12.9274) (end 30.6071 8.1654) (width 0.15) (layer "B.Cu") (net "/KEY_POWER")))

